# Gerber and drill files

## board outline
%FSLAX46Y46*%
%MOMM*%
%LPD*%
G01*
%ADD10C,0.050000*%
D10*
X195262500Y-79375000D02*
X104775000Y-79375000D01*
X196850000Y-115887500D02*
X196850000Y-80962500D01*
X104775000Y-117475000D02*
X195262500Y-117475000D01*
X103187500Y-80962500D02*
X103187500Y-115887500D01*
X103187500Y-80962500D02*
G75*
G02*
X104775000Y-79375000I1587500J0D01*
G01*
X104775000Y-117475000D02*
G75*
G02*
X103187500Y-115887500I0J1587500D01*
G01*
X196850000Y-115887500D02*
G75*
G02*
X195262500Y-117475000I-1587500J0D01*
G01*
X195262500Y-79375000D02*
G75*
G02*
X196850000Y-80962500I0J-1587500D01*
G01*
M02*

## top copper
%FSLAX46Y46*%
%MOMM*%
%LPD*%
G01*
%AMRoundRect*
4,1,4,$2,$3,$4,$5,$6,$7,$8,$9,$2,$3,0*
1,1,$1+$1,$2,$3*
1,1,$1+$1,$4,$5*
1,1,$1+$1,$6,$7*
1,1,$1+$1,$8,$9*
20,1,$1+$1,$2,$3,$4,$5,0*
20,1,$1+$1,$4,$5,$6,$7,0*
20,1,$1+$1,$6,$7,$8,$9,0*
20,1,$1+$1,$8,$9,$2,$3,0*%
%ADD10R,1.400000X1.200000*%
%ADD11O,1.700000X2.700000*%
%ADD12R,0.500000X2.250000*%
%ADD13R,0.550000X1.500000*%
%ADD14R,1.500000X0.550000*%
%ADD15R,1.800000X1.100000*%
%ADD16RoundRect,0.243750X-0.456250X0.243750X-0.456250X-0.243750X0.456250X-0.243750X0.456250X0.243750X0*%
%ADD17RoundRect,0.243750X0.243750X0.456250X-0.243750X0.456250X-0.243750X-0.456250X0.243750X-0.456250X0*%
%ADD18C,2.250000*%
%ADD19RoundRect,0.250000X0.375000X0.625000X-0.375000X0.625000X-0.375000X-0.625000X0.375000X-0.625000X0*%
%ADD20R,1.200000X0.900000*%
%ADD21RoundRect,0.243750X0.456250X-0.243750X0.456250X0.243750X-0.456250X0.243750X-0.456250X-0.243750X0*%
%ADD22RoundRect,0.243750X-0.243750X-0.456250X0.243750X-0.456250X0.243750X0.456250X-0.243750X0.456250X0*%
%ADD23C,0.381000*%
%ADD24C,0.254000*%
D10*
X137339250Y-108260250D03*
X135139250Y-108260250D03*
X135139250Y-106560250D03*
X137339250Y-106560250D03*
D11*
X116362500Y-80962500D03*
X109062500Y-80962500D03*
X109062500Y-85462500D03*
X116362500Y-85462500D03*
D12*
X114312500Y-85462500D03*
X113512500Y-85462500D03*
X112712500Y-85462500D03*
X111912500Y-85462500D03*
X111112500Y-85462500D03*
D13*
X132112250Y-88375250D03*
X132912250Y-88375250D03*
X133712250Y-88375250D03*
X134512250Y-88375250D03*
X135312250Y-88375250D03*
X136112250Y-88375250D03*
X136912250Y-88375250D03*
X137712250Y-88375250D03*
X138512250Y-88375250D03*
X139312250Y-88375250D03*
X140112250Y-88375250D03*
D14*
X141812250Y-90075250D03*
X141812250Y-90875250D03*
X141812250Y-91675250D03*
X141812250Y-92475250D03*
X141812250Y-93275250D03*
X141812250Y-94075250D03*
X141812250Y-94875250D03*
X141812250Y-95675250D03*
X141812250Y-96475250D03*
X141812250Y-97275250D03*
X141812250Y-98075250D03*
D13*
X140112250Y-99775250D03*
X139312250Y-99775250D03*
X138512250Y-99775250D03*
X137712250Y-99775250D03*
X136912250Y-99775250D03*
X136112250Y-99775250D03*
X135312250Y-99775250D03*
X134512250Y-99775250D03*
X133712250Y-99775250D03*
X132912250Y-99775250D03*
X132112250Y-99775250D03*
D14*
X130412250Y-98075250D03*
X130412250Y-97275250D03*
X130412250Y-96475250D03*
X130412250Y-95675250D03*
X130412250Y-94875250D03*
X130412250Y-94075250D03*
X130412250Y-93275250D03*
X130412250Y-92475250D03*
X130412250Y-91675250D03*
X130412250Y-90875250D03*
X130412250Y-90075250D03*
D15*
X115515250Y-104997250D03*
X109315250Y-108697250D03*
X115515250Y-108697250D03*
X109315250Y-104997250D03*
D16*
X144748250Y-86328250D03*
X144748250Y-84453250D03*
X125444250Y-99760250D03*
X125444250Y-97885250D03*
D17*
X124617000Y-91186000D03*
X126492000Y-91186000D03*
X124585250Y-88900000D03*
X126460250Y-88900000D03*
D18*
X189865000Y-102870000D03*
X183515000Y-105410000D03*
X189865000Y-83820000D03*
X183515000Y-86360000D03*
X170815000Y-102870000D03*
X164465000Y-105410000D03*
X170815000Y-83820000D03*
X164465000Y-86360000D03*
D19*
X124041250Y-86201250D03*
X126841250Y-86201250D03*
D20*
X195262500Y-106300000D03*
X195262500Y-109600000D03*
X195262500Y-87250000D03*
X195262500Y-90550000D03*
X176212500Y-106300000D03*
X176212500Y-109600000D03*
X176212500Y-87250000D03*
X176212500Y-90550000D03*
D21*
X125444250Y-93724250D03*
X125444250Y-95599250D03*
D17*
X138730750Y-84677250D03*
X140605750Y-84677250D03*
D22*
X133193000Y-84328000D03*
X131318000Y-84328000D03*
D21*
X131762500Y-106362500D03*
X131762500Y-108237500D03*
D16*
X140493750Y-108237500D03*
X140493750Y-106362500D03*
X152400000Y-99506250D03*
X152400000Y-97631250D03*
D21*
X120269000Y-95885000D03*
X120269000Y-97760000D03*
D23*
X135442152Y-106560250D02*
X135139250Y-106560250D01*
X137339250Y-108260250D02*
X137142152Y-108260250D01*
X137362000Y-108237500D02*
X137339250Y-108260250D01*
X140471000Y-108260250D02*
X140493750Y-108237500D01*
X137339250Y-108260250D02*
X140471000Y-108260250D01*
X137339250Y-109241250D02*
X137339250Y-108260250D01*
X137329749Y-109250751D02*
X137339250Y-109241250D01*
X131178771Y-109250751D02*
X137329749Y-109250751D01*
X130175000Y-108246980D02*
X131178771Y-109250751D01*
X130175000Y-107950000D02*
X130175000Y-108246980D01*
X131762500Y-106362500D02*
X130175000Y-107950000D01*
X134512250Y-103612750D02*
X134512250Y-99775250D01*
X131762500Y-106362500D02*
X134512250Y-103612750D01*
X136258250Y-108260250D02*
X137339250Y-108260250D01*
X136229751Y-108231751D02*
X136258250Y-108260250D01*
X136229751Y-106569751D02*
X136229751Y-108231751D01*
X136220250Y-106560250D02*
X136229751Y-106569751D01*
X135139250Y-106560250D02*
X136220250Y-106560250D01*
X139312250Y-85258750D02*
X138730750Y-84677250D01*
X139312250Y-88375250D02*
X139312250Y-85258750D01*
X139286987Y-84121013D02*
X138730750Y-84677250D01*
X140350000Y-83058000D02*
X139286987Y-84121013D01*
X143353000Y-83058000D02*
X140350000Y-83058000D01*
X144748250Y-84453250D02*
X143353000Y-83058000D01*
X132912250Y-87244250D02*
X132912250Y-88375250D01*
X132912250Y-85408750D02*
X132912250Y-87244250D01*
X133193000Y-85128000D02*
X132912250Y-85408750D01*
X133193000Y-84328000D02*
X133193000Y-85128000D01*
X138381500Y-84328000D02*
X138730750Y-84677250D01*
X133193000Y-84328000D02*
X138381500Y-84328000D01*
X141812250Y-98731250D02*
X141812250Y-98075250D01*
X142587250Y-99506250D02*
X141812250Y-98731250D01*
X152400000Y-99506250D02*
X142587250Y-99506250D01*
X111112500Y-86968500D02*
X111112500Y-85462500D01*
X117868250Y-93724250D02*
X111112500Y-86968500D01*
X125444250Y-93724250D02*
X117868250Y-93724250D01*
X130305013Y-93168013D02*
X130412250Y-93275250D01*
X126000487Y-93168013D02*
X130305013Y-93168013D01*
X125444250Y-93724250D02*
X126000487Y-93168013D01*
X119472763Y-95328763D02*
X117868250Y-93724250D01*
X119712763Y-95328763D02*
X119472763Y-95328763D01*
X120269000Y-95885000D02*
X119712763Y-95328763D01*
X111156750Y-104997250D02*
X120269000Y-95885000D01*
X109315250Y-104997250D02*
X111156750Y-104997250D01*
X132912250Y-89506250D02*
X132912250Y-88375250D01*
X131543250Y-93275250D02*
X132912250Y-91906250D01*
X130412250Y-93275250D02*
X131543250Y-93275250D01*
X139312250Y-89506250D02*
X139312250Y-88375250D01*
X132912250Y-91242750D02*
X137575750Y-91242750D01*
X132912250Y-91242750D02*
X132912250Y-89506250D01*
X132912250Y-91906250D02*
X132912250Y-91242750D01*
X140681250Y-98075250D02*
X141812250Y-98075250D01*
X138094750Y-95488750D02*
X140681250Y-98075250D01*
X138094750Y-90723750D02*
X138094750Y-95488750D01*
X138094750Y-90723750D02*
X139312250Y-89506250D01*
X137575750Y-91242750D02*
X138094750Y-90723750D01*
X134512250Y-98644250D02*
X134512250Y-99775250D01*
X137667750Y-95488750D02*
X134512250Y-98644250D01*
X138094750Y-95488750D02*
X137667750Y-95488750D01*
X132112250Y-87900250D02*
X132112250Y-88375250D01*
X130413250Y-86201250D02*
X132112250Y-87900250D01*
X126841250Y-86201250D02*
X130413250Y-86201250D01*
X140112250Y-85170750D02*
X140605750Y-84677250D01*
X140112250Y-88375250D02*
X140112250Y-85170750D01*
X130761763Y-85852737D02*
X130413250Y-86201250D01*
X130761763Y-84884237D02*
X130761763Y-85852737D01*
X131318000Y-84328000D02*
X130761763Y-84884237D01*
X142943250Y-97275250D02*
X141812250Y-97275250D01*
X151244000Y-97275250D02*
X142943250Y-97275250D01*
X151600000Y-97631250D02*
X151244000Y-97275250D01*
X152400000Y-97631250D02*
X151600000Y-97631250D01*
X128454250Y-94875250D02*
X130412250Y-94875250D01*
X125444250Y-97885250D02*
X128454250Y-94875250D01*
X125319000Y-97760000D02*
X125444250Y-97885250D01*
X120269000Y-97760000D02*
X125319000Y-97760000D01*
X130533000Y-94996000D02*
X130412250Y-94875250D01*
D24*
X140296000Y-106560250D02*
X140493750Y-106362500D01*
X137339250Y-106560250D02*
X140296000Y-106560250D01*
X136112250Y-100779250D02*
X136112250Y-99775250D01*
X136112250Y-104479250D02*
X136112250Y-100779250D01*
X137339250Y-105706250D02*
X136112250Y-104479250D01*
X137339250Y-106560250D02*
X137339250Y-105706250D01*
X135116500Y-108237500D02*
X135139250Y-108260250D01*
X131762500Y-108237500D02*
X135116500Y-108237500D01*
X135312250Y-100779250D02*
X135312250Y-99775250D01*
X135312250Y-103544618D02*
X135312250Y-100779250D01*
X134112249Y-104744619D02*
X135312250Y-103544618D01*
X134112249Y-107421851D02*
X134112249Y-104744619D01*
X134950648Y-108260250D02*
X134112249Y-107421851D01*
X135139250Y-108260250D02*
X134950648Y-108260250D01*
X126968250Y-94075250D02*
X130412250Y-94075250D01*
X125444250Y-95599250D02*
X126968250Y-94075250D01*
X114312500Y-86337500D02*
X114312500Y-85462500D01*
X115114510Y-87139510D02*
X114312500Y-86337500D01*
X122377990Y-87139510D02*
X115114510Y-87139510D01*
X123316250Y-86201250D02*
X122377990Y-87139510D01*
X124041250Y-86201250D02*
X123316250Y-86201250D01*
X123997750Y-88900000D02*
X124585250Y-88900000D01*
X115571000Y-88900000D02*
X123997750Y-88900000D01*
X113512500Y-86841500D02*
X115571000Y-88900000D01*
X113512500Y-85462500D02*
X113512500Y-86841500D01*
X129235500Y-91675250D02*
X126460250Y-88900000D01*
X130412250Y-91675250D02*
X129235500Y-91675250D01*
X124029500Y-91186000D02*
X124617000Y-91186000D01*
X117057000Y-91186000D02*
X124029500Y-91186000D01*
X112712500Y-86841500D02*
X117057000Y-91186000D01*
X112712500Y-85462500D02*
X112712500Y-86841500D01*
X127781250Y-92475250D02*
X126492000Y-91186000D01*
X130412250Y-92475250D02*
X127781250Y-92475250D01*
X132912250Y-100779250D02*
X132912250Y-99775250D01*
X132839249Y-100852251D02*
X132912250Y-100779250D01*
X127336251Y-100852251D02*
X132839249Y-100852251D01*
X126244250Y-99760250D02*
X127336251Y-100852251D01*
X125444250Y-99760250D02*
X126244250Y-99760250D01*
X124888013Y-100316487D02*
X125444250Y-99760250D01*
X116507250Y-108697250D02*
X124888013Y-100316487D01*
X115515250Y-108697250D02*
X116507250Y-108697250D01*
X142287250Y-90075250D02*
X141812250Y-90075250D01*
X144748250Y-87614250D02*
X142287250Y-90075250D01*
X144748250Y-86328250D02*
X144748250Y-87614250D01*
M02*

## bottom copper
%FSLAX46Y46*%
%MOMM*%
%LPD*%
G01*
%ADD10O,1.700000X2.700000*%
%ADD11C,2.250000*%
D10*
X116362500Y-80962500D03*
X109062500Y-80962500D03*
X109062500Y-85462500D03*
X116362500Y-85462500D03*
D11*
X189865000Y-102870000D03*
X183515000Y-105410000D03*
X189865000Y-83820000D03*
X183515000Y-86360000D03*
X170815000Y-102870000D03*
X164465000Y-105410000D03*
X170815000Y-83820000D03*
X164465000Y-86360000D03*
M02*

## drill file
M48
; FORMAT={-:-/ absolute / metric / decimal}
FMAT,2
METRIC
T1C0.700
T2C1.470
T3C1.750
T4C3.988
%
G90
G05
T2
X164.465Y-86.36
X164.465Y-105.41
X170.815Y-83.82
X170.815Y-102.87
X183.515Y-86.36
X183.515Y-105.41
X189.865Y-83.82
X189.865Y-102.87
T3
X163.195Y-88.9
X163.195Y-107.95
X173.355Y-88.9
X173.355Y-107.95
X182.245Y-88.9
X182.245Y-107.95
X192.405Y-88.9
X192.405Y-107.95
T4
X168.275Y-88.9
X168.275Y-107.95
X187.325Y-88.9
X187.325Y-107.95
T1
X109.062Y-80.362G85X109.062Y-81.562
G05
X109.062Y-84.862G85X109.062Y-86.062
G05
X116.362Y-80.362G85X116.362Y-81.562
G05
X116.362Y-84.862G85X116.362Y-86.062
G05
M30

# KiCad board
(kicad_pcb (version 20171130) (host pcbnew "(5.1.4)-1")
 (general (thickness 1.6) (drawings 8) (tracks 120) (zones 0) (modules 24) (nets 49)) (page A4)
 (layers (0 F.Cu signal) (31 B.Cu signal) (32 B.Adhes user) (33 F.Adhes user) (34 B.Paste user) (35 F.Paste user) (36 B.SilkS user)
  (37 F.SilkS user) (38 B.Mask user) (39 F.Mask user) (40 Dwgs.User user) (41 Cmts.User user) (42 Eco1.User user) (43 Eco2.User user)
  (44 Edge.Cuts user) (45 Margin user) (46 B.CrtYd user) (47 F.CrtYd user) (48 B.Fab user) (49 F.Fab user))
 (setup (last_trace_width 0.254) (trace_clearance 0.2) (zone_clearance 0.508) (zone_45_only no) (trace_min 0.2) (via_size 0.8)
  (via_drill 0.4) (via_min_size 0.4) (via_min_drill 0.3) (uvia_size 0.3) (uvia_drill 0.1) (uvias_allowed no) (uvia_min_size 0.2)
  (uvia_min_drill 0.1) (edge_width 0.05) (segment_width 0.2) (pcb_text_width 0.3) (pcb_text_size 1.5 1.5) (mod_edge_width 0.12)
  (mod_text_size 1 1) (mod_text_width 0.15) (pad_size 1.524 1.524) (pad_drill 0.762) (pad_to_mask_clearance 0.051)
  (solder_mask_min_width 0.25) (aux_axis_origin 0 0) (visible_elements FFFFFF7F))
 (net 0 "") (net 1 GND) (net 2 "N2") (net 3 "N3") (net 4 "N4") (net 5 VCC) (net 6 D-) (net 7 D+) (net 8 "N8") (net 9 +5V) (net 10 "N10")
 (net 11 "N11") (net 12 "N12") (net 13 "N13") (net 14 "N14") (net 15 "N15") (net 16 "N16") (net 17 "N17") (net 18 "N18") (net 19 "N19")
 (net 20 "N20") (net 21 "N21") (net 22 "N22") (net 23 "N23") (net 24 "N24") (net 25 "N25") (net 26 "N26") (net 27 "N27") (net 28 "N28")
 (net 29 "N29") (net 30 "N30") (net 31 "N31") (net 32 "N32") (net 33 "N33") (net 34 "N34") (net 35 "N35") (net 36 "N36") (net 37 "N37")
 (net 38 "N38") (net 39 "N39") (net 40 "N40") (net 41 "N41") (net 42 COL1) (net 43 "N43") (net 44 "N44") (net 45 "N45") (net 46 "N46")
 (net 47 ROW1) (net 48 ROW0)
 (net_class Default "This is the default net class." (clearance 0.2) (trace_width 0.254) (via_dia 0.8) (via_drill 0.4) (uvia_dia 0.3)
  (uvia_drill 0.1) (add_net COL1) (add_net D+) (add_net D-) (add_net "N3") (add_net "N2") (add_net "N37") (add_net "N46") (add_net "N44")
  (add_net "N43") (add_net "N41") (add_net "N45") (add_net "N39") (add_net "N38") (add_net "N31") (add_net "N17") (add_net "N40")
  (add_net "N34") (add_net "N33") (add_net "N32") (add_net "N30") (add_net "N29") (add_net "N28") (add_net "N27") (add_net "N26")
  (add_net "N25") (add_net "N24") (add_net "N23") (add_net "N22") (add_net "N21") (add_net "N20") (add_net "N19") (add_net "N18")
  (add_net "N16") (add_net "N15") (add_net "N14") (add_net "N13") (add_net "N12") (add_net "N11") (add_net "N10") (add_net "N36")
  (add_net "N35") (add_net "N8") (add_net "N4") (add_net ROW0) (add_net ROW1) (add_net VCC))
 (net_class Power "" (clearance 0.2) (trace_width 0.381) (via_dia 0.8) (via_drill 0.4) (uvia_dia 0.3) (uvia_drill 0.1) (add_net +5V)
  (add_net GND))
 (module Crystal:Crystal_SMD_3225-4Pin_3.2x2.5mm (layer F.Cu) (at 136.23925 107.41025 180)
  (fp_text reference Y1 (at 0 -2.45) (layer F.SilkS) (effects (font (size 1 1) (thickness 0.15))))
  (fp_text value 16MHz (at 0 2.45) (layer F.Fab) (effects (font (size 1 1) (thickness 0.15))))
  (pad 4 smd rect (at -1.1 -0.85 180) (size 1.4 1.2) (layers F.Cu F.Paste F.Mask) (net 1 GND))
  (pad 3 smd rect (at 1.1 -0.85 180) (size 1.4 1.2) (layers F.Cu F.Paste F.Mask) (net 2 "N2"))
  (pad 2 smd rect (at 1.1 0.85 180) (size 1.4 1.2) (layers F.Cu F.Paste F.Mask) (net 1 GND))
  (pad 1 smd rect (at -1.1 0.85 180) (size 1.4 1.2) (layers F.Cu F.Paste F.Mask) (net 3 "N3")))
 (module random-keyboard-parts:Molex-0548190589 (layer F.Cu) (at 112.7125 80.9625 270)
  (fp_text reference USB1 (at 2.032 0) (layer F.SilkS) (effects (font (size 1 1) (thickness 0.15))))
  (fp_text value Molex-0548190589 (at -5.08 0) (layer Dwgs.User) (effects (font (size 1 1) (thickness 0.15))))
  (pad 6 thru_hole oval (at 0 -3.65 270) (size 2.7 1.7) (drill oval 1.9 0.7) (layers *.Cu *.Mask) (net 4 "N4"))
  (pad 6 thru_hole oval (at 0 3.65 270) (size 2.7 1.7) (drill oval 1.9 0.7) (layers *.Cu *.Mask) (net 4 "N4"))
  (pad 6 thru_hole oval (at 4.5 3.65 270) (size 2.7 1.7) (drill oval 1.9 0.7) (layers *.Cu *.Mask) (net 4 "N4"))
  (pad 6 thru_hole oval (at 4.5 -3.65 270) (size 2.7 1.7) (drill oval 1.9 0.7) (layers *.Cu *.Mask) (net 4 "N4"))
  (pad 5 smd rect (at 4.5 -1.6 270) (size 2.25 0.5) (layers F.Cu F.Paste F.Mask) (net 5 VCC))
  (pad 4 smd rect (at 4.5 -0.8 270) (size 2.25 0.5) (layers F.Cu F.Paste F.Mask) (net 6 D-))
  (pad 3 smd rect (at 4.5 0 270) (size 2.25 0.5) (layers F.Cu F.Paste F.Mask) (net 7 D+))
  (pad 2 smd rect (at 4.5 0.8 270) (size 2.25 0.5) (layers F.Cu F.Paste F.Mask) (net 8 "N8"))
  (pad 1 smd rect (at 4.5 1.6 270) (size 2.25 0.5) (layers F.Cu F.Paste F.Mask) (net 1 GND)))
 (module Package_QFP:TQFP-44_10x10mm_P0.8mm (layer F.Cu) (at 136.11225 94.07525)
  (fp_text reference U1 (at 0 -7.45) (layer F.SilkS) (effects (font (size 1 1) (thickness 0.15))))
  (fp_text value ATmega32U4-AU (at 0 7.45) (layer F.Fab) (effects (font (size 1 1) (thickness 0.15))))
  (pad 44 smd rect (at -4 -5.7 90) (size 1.5 0.55) (layers F.Cu F.Paste F.Mask) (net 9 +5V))
  (pad 43 smd rect (at -3.2 -5.7 90) (size 1.5 0.55) (layers F.Cu F.Paste F.Mask) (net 1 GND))
  (pad 42 smd rect (at -2.4 -5.7 90) (size 1.5 0.55) (layers F.Cu F.Paste F.Mask) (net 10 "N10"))
  (pad 41 smd rect (at -1.6 -5.7 90) (size 1.5 0.55) (layers F.Cu F.Paste F.Mask) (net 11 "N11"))
  (pad 40 smd rect (at -0.8 -5.7 90) (size 1.5 0.55) (layers F.Cu F.Paste F.Mask) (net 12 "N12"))
  (pad 39 smd rect (at 0 -5.7 90) (size 1.5 0.55) (layers F.Cu F.Paste F.Mask) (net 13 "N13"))
  (pad 38 smd rect (at 0.8 -5.7 90) (size 1.5 0.55) (layers F.Cu F.Paste F.Mask) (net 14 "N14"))
  (pad 37 smd rect (at 1.6 -5.7 90) (size 1.5 0.55) (layers F.Cu F.Paste F.Mask) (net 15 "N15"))
  (pad 36 smd rect (at 2.4 -5.7 90) (size 1.5 0.55) (layers F.Cu F.Paste F.Mask) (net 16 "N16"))
  (pad 35 smd rect (at 3.2 -5.7 90) (size 1.5 0.55) (layers F.Cu F.Paste F.Mask) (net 1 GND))
  (pad 34 smd rect (at 4 -5.7 90) (size 1.5 0.55) (layers F.Cu F.Paste F.Mask) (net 9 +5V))
  (pad 33 smd rect (at 5.7 -4) (size 1.5 0.55) (layers F.Cu F.Paste F.Mask) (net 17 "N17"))
  (pad 32 smd rect (at 5.7 -3.2) (size 1.5 0.55) (layers F.Cu F.Paste F.Mask) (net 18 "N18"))
  (pad 31 smd rect (at 5.7 -2.4) (size 1.5 0.55) (layers F.Cu F.Paste F.Mask) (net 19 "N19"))
  (pad 30 smd rect (at 5.7 -1.6) (size 1.5 0.55) (layers F.Cu F.Paste F.Mask) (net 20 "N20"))
  (pad 29 smd rect (at 5.7 -0.8) (size 1.5 0.55) (layers F.Cu F.Paste F.Mask) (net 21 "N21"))
  (pad 28 smd rect (at 5.7 0) (size 1.5 0.55) (layers F.Cu F.Paste F.Mask) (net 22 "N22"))
  (pad 27 smd rect (at 5.7 0.8) (size 1.5 0.55) (layers F.Cu F.Paste F.Mask) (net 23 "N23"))
  (pad 26 smd rect (at 5.7 1.6) (size 1.5 0.55) (layers F.Cu F.Paste F.Mask) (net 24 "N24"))
  (pad 25 smd rect (at 5.7 2.4) (size 1.5 0.55) (layers F.Cu F.Paste F.Mask) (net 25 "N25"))
  (pad 24 smd rect (at 5.7 3.2) (size 1.5 0.55) (layers F.Cu F.Paste F.Mask) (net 9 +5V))
  (pad 23 smd rect (at 5.7 4) (size 1.5 0.55) (layers F.Cu F.Paste F.Mask) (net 1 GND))
  (pad 22 smd rect (at 4 5.7 90) (size 1.5 0.55) (layers F.Cu F.Paste F.Mask) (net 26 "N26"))
  (pad 21 smd rect (at 3.2 5.7 90) (size 1.5 0.55) (layers F.Cu F.Paste F.Mask) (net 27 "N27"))
  (pad 20 smd rect (at 2.4 5.7 90) (size 1.5 0.55) (layers F.Cu F.Paste F.Mask) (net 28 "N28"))
  (pad 19 smd rect (at 1.6 5.7 90) (size 1.5 0.55) (layers F.Cu F.Paste F.Mask) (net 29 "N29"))
  (pad 18 smd rect (at 0.8 5.7 90) (size 1.5 0.55) (layers F.Cu F.Paste F.Mask) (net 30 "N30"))
  (pad 17 smd rect (at 0 5.7 90) (size 1.5 0.55) (layers F.Cu F.Paste F.Mask) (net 3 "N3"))
  (pad 16 smd rect (at -0.8 5.7 90) (size 1.5 0.55) (layers F.Cu F.Paste F.Mask) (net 2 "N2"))
  (pad 15 smd rect (at -1.6 5.7 90) (size 1.5 0.55) (layers F.Cu F.Paste F.Mask) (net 1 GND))
  (pad 14 smd rect (at -2.4 5.7 90) (size 1.5 0.55) (layers F.Cu F.Paste F.Mask) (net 9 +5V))
  (pad 13 smd rect (at -3.2 5.7 90) (size 1.5 0.55) (layers F.Cu F.Paste F.Mask) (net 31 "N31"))
  (pad 12 smd rect (at -4 5.7 90) (size 1.5 0.55) (layers F.Cu F.Paste F.Mask) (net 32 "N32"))
  (pad 11 smd rect (at -5.7 4) (size 1.5 0.55) (layers F.Cu F.Paste F.Mask) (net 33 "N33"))
  (pad 10 smd rect (at -5.7 3.2) (size 1.5 0.55) (layers F.Cu F.Paste F.Mask) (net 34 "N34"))
  (pad 9 smd rect (at -5.7 2.4) (size 1.5 0.55) (layers F.Cu F.Paste F.Mask) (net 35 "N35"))
  (pad 8 smd rect (at -5.7 1.6) (size 1.5 0.55) (layers F.Cu F.Paste F.Mask) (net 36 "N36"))
  (pad 7 smd rect (at -5.7 0.8) (size 1.5 0.55) (layers F.Cu F.Paste F.Mask) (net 9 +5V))
  (pad 6 smd rect (at -5.7 0) (size 1.5 0.55) (layers F.Cu F.Paste F.Mask) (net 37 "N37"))
  (pad 5 smd rect (at -5.7 -0.8) (size 1.5 0.55) (layers F.Cu F.Paste F.Mask) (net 1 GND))
  (pad 4 smd rect (at -5.7 -1.6) (size 1.5 0.55) (layers F.Cu F.Paste F.Mask) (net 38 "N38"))
  (pad 3 smd rect (at -5.7 -2.4) (size 1.5 0.55) (layers F.Cu F.Paste F.Mask) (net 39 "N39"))
  (pad 2 smd rect (at -5.7 -3.2) (size 1.5 0.55) (layers F.Cu F.Paste F.Mask) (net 9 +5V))
  (pad 1 smd rect (at -5.7 -4) (size 1.5 0.55) (layers F.Cu F.Paste F.Mask) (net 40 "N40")))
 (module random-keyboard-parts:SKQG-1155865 (layer F.Cu) (at 112.41525 106.84725 180)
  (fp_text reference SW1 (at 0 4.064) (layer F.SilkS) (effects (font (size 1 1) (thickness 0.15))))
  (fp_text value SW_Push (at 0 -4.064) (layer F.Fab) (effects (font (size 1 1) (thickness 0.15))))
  (pad 4 smd rect (at -3.1 1.85 180) (size 1.8 1.1) (layers F.Cu F.Paste F.Mask))
  (pad 3 smd rect (at 3.1 -1.85 180) (size 1.8 1.1) (layers F.Cu F.Paste F.Mask))
  (pad 2 smd rect (at -3.1 -1.85 180) (size 1.8 1.1) (layers F.Cu F.Paste F.Mask) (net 31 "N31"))
  (pad 1 smd rect (at 3.1 1.85 180) (size 1.8 1.1) (layers F.Cu F.Paste F.Mask) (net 1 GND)))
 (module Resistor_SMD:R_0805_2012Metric (layer F.Cu) (at 144.74825 85.39075 270)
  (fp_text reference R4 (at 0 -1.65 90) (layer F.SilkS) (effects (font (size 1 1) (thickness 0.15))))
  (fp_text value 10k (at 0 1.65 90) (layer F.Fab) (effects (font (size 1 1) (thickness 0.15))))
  (pad 2 smd roundrect (at 0.9375 0 270) (size 0.975 1.4) (layers F.Cu F.Paste F.Mask) (roundrect_rratio 0.25) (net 17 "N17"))
  (pad 1 smd roundrect (at -0.9375 0 270) (size 0.975 1.4) (layers F.Cu F.Paste F.Mask) (roundrect_rratio 0.25) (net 1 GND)))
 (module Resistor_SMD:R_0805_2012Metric (layer F.Cu) (at 125.44425 98.82275 270)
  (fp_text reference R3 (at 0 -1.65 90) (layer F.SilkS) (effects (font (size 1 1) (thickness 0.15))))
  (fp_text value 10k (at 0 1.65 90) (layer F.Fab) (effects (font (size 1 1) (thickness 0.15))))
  (pad 2 smd roundrect (at 0.9375 0 270) (size 0.975 1.4) (layers F.Cu F.Paste F.Mask) (roundrect_rratio 0.25) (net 31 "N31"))
  (pad 1 smd roundrect (at -0.9375 0 270) (size 0.975 1.4) (layers F.Cu F.Paste F.Mask) (roundrect_rratio 0.25) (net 9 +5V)))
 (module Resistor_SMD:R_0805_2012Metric (layer F.Cu) (at 125.5545 91.186 180)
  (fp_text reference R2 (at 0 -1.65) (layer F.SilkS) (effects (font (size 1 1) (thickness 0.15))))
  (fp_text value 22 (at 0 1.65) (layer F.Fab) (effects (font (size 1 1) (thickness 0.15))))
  (pad 2 smd roundrect (at 0.9375 0 180) (size 0.975 1.4) (layers F.Cu F.Paste F.Mask) (roundrect_rratio 0.25) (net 7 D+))
  (pad 1 smd roundrect (at -0.9375 0 180) (size 0.975 1.4) (layers F.Cu F.Paste F.Mask) (roundrect_rratio 0.25) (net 38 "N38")))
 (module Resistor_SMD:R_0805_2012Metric (layer F.Cu) (at 125.52275 88.9 180)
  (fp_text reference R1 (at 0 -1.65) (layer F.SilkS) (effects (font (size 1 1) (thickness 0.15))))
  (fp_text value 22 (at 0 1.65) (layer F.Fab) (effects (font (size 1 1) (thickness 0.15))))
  (pad 2 smd roundrect (at 0.9375 0 180) (size 0.975 1.4) (layers F.Cu F.Paste F.Mask) (roundrect_rratio 0.25) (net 6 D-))
  (pad 1 smd roundrect (at -0.9375 0 180) (size 0.975 1.4) (layers F.Cu F.Paste F.Mask) (roundrect_rratio 0.25) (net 39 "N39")))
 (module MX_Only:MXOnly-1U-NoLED (layer F.Cu) (at 187.325 107.95)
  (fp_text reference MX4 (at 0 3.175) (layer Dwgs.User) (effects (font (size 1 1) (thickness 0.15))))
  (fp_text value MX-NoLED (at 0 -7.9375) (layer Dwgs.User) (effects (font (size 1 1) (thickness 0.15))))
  (pad 2 thru_hole circle (at 2.54 -5.08) (size 2.25 2.25) (drill 1.47) (layers *.Cu B.Mask) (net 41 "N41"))
  (pad "" np_thru_hole circle (at 0 0) (size 3.9878 3.9878) (drill 3.9878) (layers *.Cu *.Mask))
  (pad 1 thru_hole circle (at -3.81 -2.54) (size 2.25 2.25) (drill 1.47) (layers *.Cu B.Mask) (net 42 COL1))
  (pad "" np_thru_hole circle (at -5.08 0 48.0996) (size 1.75 1.75) (drill 1.75) (layers *.Cu *.Mask))
  (pad "" np_thru_hole circle (at 5.08 0 48.0996) (size 1.75 1.75) (drill 1.75) (layers *.Cu *.Mask)))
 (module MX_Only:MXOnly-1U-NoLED (layer F.Cu) (at 187.325 88.9)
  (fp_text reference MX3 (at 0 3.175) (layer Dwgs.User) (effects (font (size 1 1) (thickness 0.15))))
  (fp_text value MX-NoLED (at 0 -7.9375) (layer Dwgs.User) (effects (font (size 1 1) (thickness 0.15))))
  (pad 2 thru_hole circle (at 2.54 -5.08) (size 2.25 2.25) (drill 1.47) (layers *.Cu B.Mask) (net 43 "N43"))
  (pad "" np_thru_hole circle (at 0 0) (size 3.9878 3.9878) (drill 3.9878) (layers *.Cu *.Mask))
  (pad 1 thru_hole circle (at -3.81 -2.54) (size 2.25 2.25) (drill 1.47) (layers *.Cu B.Mask) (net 42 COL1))
  (pad "" np_thru_hole circle (at -5.08 0 48.0996) (size 1.75 1.75) (drill 1.75) (layers *.Cu *.Mask))
  (pad "" np_thru_hole circle (at 5.08 0 48.0996) (size 1.75 1.75) (drill 1.75) (layers *.Cu *.Mask)))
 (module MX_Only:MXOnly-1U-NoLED (layer F.Cu) (at 168.275 107.95)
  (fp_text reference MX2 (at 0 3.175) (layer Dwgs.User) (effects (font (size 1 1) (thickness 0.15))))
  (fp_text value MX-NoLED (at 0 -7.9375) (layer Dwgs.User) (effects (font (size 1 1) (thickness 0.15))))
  (pad 2 thru_hole circle (at 2.54 -5.08) (size 2.25 2.25) (drill 1.47) (layers *.Cu B.Mask) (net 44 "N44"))
  (pad "" np_thru_hole circle (at 0 0) (size 3.9878 3.9878) (drill 3.9878) (layers *.Cu *.Mask))
  (pad 1 thru_hole circle (at -3.81 -2.54) (size 2.25 2.25) (drill 1.47) (layers *.Cu B.Mask) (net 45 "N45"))
  (pad "" np_thru_hole circle (at -5.08 0 48.0996) (size 1.75 1.75) (drill 1.75) (layers *.Cu *.Mask))
  (pad "" np_thru_hole circle (at 5.08 0 48.0996) (size 1.75 1.75) (drill 1.75) (layers *.Cu *.Mask)))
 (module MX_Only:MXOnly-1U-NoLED (layer F.Cu) (at 168.275 88.9)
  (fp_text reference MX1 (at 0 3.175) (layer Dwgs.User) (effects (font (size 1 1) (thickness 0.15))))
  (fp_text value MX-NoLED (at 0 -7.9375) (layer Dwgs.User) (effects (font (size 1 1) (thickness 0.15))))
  (pad 2 thru_hole circle (at 2.54 -5.08) (size 2.25 2.25) (drill 1.47) (layers *.Cu B.Mask) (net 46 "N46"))
  (pad "" np_thru_hole circle (at 0 0) (size 3.9878 3.9878) (drill 3.9878) (layers *.Cu *.Mask))
  (pad 1 thru_hole circle (at -3.81 -2.54) (size 2.25 2.25) (drill 1.47) (layers *.Cu B.Mask) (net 45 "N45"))
  (pad "" np_thru_hole circle (at -5.08 0 48.0996) (size 1.75 1.75) (drill 1.75) (layers *.Cu *.Mask))
  (pad "" np_thru_hole circle (at 5.08 0 48.0996) (size 1.75 1.75) (drill 1.75) (layers *.Cu *.Mask)))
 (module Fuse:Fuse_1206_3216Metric (layer F.Cu) (at 125.44125 86.20125 180)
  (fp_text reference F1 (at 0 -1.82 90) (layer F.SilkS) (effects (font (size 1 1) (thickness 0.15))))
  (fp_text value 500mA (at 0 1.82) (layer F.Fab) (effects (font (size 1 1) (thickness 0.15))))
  (pad 2 smd roundrect (at 1.4 0 180) (size 1.25 1.75) (layers F.Cu F.Paste F.Mask) (roundrect_rratio 0.2) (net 5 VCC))
  (pad 1 smd roundrect (at -1.4 0 180) (size 1.25 1.75) (layers F.Cu F.Paste F.Mask) (roundrect_rratio 0.2) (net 9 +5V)))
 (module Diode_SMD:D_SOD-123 (layer F.Cu) (at 195.2625 107.95 90)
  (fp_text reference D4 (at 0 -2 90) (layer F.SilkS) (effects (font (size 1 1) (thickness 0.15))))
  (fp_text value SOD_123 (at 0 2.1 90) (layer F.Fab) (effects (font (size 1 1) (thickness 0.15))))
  (pad 2 smd rect (at 1.65 0 90) (size 0.9 1.2) (layers F.Cu F.Paste F.Mask) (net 41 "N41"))
  (pad 1 smd rect (at -1.65 0 90) (size 0.9 1.2) (layers F.Cu F.Paste F.Mask) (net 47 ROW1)))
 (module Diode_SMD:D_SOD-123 (layer F.Cu) (at 195.2625 88.9 90)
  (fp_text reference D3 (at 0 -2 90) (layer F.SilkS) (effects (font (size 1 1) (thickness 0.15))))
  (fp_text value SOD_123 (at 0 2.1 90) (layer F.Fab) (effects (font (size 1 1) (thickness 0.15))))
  (pad 2 smd rect (at 1.65 0 90) (size 0.9 1.2) (layers F.Cu F.Paste F.Mask) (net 43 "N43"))
  (pad 1 smd rect (at -1.65 0 90) (size 0.9 1.2) (layers F.Cu F.Paste F.Mask) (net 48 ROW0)))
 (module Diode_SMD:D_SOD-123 (layer F.Cu) (at 176.2125 107.95 90)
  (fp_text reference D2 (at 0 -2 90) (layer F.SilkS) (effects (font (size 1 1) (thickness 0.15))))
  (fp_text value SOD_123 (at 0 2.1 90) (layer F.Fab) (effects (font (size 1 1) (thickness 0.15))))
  (pad 2 smd rect (at 1.65 0 90) (size 0.9 1.2) (layers F.Cu F.Paste F.Mask) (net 44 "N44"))
  (pad 1 smd rect (at -1.65 0 90) (size 0.9 1.2) (layers F.Cu F.Paste F.Mask) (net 47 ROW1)))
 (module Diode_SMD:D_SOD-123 (layer F.Cu) (at 176.2125 88.9 90)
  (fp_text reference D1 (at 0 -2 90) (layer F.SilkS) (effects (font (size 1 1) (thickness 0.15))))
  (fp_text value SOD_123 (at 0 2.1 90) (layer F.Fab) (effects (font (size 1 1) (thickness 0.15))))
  (pad 2 smd rect (at 1.65 0 90) (size 0.9 1.2) (layers F.Cu F.Paste F.Mask) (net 46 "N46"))
  (pad 1 smd rect (at -1.65 0 90) (size 0.9 1.2) (layers F.Cu F.Paste F.Mask) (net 48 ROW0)))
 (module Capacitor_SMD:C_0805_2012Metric (layer F.Cu) (at 125.44425 94.66175 90)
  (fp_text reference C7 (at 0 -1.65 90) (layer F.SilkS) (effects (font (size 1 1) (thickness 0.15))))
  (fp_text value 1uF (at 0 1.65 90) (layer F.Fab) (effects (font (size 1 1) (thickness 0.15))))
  (pad 2 smd roundrect (at 0.9375 0 90) (size 0.975 1.4) (layers F.Cu F.Paste F.Mask) (roundrect_rratio 0.25) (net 1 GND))
  (pad 1 smd roundrect (at -0.9375 0 90) (size 0.975 1.4) (layers F.Cu F.Paste F.Mask) (roundrect_rratio 0.25) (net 37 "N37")))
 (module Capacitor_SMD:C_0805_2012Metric (layer F.Cu) (at 139.66825 84.67725 180)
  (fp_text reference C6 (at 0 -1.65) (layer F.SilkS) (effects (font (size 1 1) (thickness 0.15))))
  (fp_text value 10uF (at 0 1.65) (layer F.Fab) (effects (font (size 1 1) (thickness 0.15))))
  (pad 2 smd roundrect (at 0.9375 0 180) (size 0.975 1.4) (layers F.Cu F.Paste F.Mask) (roundrect_rratio 0.25) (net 1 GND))
  (pad 1 smd roundrect (at -0.9375 0 180) (size 0.975 1.4) (layers F.Cu F.Paste F.Mask) (roundrect_rratio 0.25) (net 9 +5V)))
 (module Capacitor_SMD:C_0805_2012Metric (layer F.Cu) (at 132.2555 84.328)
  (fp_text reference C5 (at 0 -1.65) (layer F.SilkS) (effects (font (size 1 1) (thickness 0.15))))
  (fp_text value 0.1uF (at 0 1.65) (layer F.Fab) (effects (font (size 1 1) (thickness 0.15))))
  (pad 2 smd roundrect (at 0.9375 0) (size 0.975 1.4) (layers F.Cu F.Paste F.Mask) (roundrect_rratio 0.25) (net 1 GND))
  (pad 1 smd roundrect (at -0.9375 0) (size 0.975 1.4) (layers F.Cu F.Paste F.Mask) (roundrect_rratio 0.25) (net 9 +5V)))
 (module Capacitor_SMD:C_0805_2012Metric (layer F.Cu) (at 131.7625 107.3 90)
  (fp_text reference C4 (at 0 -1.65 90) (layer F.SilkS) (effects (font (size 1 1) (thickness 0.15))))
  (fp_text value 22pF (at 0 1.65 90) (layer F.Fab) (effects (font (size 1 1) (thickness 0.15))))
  (pad 2 smd roundrect (at 0.9375 0 90) (size 0.975 1.4) (layers F.Cu F.Paste F.Mask) (roundrect_rratio 0.25) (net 1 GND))
  (pad 1 smd roundrect (at -0.9375 0 90) (size 0.975 1.4) (layers F.Cu F.Paste F.Mask) (roundrect_rratio 0.25) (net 2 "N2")))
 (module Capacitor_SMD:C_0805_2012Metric (layer F.Cu) (at 140.49375 107.3 270)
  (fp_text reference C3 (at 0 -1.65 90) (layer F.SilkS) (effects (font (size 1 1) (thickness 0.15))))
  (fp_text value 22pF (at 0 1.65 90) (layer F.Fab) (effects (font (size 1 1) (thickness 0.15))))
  (pad 2 smd roundrect (at 0.9375 0 270) (size 0.975 1.4) (layers F.Cu F.Paste F.Mask) (roundrect_rratio 0.25) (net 1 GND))
  (pad 1 smd roundrect (at -0.9375 0 270) (size 0.975 1.4) (layers F.Cu F.Paste F.Mask) (roundrect_rratio 0.25) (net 3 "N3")))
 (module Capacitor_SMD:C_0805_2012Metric (layer F.Cu) (at 152.4 98.56875 270)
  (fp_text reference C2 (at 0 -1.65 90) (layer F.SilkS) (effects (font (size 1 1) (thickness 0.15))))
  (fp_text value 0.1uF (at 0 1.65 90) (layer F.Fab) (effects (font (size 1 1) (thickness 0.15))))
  (pad 2 smd roundrect (at 0.9375 0 270) (size 0.975 1.4) (layers F.Cu F.Paste F.Mask) (roundrect_rratio 0.25) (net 1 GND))
  (pad 1 smd roundrect (at -0.9375 0 270) (size 0.975 1.4) (layers F.Cu F.Paste F.Mask) (roundrect_rratio 0.25) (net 9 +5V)))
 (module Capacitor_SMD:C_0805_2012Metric (layer F.Cu) (at 120.269 96.8225 90)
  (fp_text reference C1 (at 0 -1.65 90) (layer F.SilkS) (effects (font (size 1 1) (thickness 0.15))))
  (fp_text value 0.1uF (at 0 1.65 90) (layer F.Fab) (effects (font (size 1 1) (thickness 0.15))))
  (pad 2 smd roundrect (at 0.9375 0 90) (size 0.975 1.4) (layers F.Cu F.Paste F.Mask) (roundrect_rratio 0.25) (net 1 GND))
  (pad 1 smd roundrect (at -0.9375 0 90) (size 0.975 1.4) (layers F.Cu F.Paste F.Mask) (roundrect_rratio 0.25) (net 9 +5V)))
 (gr_line (start 195.2625 79.375) (end 104.775 79.375) (layer Edge.Cuts) (width 0.05))
 (gr_line (start 196.85 115.8875) (end 196.85 80.9625) (layer Edge.Cuts) (width 0.05))
 (gr_line (start 104.775 117.475) (end 195.2625 117.475) (layer Edge.Cuts) (width 0.05))
 (gr_line (start 103.1875 80.9625) (end 103.1875 115.8875) (layer Edge.Cuts) (width 0.05))
 (gr_arc (start 104.775 80.9625) (end 104.775 79.375) (angle -90) (layer Edge.Cuts) (width 0.05))
 (gr_arc (start 104.775 115.8875) (end 103.1875 115.8875) (angle -90) (layer Edge.Cuts) (width 0.05))
 (gr_arc (start 195.2625 115.8875) (end 195.2625 117.475) (angle -90) (layer Edge.Cuts) (width 0.05))
 (gr_arc (start 195.2625 80.9625) (end 196.85 80.9625) (angle -90) (layer Edge.Cuts) (width 0.05))
 (segment (start 135.442152 106.56025) (end 135.13925 106.56025) (width 0.381) (layer F.Cu) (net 1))
 (segment (start 137.33925 108.26025) (end 137.142152 108.26025) (width 0.381) (layer F.Cu) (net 1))
 (segment (start 137.362 108.2375) (end 137.33925 108.26025) (width 0.381) (layer F.Cu) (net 1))
 (segment (start 140.471 108.26025) (end 140.49375 108.2375) (width 0.381) (layer F.Cu) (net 1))
 (segment (start 137.33925 108.26025) (end 140.471 108.26025) (width 0.381) (layer F.Cu) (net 1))
 (segment (start 137.33925 109.24125) (end 137.33925 108.26025) (width 0.381) (layer F.Cu) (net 1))
 (segment (start 137.329749 109.250751) (end 137.33925 109.24125) (width 0.381) (layer F.Cu) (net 1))
 (segment (start 131.178771 109.250751) (end 137.329749 109.250751) (width 0.381) (layer F.Cu) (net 1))
 (segment (start 130.175 108.24698) (end 131.178771 109.250751) (width 0.381) (layer F.Cu) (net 1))
 (segment (start 130.175 107.95) (end 130.175 108.24698) (width 0.381) (layer F.Cu) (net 1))
 (segment (start 131.7625 106.3625) (end 130.175 107.95) (width 0.381) (layer F.Cu) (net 1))
 (segment (start 134.51225 103.61275) (end 134.51225 99.77525) (width 0.381) (layer F.Cu) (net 1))
 (segment (start 131.7625 106.3625) (end 134.51225 103.61275) (width 0.381) (layer F.Cu) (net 1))
 (segment (start 136.25825 108.26025) (end 137.33925 108.26025) (width 0.381) (layer F.Cu) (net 1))
 (segment (start 136.229751 108.231751) (end 136.25825 108.26025) (width 0.381) (layer F.Cu) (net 1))
 (segment (start 136.229751 106.569751) (end 136.229751 108.231751) (width 0.381) (layer F.Cu) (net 1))
 (segment (start 136.22025 106.56025) (end 136.229751 106.569751) (width 0.381) (layer F.Cu) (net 1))
 (segment (start 135.13925 106.56025) (end 136.22025 106.56025) (width 0.381) (layer F.Cu) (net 1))
 (segment (start 139.31225 85.25875) (end 138.73075 84.67725) (width 0.381) (layer F.Cu) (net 1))
 (segment (start 139.31225 88.37525) (end 139.31225 85.25875) (width 0.381) (layer F.Cu) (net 1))
 (segment (start 139.286987 84.121013) (end 138.73075 84.67725) (width 0.381) (layer F.Cu) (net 1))
 (segment (start 140.35 83.058) (end 139.286987 84.121013) (width 0.381) (layer F.Cu) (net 1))
 (segment (start 143.353 83.058) (end 140.35 83.058) (width 0.381) (layer F.Cu) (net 1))
 (segment (start 144.74825 84.45325) (end 143.353 83.058) (width 0.381) (layer F.Cu) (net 1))
 (segment (start 132.91225 87.24425) (end 132.91225 88.37525) (width 0.381) (layer F.Cu) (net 1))
 (segment (start 132.91225 85.40875) (end 132.91225 87.24425) (width 0.381) (layer F.Cu) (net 1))
 (segment (start 133.193 85.128) (end 132.91225 85.40875) (width 0.381) (layer F.Cu) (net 1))
 (segment (start 133.193 84.328) (end 133.193 85.128) (width 0.381) (layer F.Cu) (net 1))
 (segment (start 138.3815 84.328) (end 138.73075 84.67725) (width 0.381) (layer F.Cu) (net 1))
 (segment (start 133.193 84.328) (end 138.3815 84.328) (width 0.381) (layer F.Cu) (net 1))
 (segment (start 141.81225 98.73125) (end 141.81225 98.07525) (width 0.381) (layer F.Cu) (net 1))
 (segment (start 142.58725 99.50625) (end 141.81225 98.73125) (width 0.381) (layer F.Cu) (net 1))
 (segment (start 152.4 99.50625) (end 142.58725 99.50625) (width 0.381) (layer F.Cu) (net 1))
 (segment (start 111.1125 86.9685) (end 111.1125 85.4625) (width 0.381) (layer F.Cu) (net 1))
 (segment (start 117.86825 93.72425) (end 111.1125 86.9685) (width 0.381) (layer F.Cu) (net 1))
 (segment (start 125.44425 93.72425) (end 117.86825 93.72425) (width 0.381) (layer F.Cu) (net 1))
 (segment (start 130.305013 93.168013) (end 130.41225 93.27525) (width 0.381) (layer F.Cu) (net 1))
 (segment (start 126.000487 93.168013) (end 130.305013 93.168013) (width 0.381) (layer F.Cu) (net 1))
 (segment (start 125.44425 93.72425) (end 126.000487 93.168013) (width 0.381) (layer F.Cu) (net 1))
 (segment (start 119.472763 95.328763) (end 117.86825 93.72425) (width 0.381) (layer F.Cu) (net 1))
 (segment (start 119.712763 95.328763) (end 119.472763 95.328763) (width 0.381) (layer F.Cu) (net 1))
 (segment (start 120.269 95.885) (end 119.712763 95.328763) (width 0.381) (layer F.Cu) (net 1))
 (segment (start 111.15675 104.99725) (end 120.269 95.885) (width 0.381) (layer F.Cu) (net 1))
 (segment (start 109.31525 104.99725) (end 111.15675 104.99725) (width 0.381) (layer F.Cu) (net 1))
 (segment (start 132.91225 89.50625) (end 132.91225 88.37525) (width 0.381) (layer F.Cu) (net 1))
 (segment (start 131.54325 93.27525) (end 132.91225 91.90625) (width 0.381) (layer F.Cu) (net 1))
 (segment (start 130.41225 93.27525) (end 131.54325 93.27525) (width 0.381) (layer F.Cu) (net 1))
 (segment (start 139.31225 89.50625) (end 139.31225 88.37525) (width 0.381) (layer F.Cu) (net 1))
 (segment (start 132.91225 91.24275) (end 137.57575 91.24275) (width 0.381) (layer F.Cu) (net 1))
 (segment (start 132.91225 91.24275) (end 132.91225 89.50625) (width 0.381) (layer F.Cu) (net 1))
 (segment (start 132.91225 91.90625) (end 132.91225 91.24275) (width 0.381) (layer F.Cu) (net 1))
 (segment (start 140.68125 98.07525) (end 141.81225 98.07525) (width 0.381) (layer F.Cu) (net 1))
 (segment (start 138.09475 95.48875) (end 140.68125 98.07525) (width 0.381) (layer F.Cu) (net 1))
 (segment (start 138.09475 90.72375) (end 138.09475 95.48875) (width 0.381) (layer F.Cu) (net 1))
 (segment (start 138.09475 90.72375) (end 139.31225 89.50625) (width 0.381) (layer F.Cu) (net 1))
 (segment (start 137.57575 91.24275) (end 138.09475 90.72375) (width 0.381) (layer F.Cu) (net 1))
 (segment (start 134.51225 98.64425) (end 134.51225 99.77525) (width 0.381) (layer F.Cu) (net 1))
 (segment (start 137.66775 95.48875) (end 134.51225 98.64425) (width 0.381) (layer F.Cu) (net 1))
 (segment (start 138.09475 95.48875) (end 137.66775 95.48875) (width 0.381) (layer F.Cu) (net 1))
 (segment (start 132.11225 87.90025) (end 132.11225 88.37525) (width 0.381) (layer F.Cu) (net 9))
 (segment (start 130.41325 86.20125) (end 132.11225 87.90025) (width 0.381) (layer F.Cu) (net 9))
 (segment (start 126.84125 86.20125) (end 130.41325 86.20125) (width 0.381) (layer F.Cu) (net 9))
 (segment (start 140.11225 85.17075) (end 140.60575 84.67725) (width 0.381) (layer F.Cu) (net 9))
 (segment (start 140.11225 88.37525) (end 140.11225 85.17075) (width 0.381) (layer F.Cu) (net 9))
 (segment (start 130.761763 85.852737) (end 130.41325 86.20125) (width 0.381) (layer F.Cu) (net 9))
 (segment (start 130.761763 84.884237) (end 130.761763 85.852737) (width 0.381) (layer F.Cu) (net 9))
 (segment (start 131.318 84.328) (end 130.761763 84.884237) (width 0.381) (layer F.Cu) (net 9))
 (segment (start 142.94325 97.27525) (end 141.81225 97.27525) (width 0.381) (layer F.Cu) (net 9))
 (segment (start 151.244 97.27525) (end 142.94325 97.27525) (width 0.381) (layer F.Cu) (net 9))
 (segment (start 151.6 97.63125) (end 151.244 97.27525) (width 0.381) (layer F.Cu) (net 9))
 (segment (start 152.4 97.63125) (end 151.6 97.63125) (width 0.381) (layer F.Cu) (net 9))
 (segment (start 128.45425 94.87525) (end 130.41225 94.87525) (width 0.381) (layer F.Cu) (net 9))
 (segment (start 125.44425 97.88525) (end 128.45425 94.87525) (width 0.381) (layer F.Cu) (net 9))
 (segment (start 125.319 97.76) (end 125.44425 97.88525) (width 0.381) (layer F.Cu) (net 9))
 (segment (start 120.269 97.76) (end 125.319 97.76) (width 0.381) (layer F.Cu) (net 9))
 (segment (start 130.533 94.996) (end 130.41225 94.87525) (width 0.381) (layer F.Cu) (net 9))
 (segment (start 140.296 106.56025) (end 140.49375 106.3625) (width 0.254) (layer F.Cu) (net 3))
 (segment (start 137.33925 106.56025) (end 140.296 106.56025) (width 0.254) (layer F.Cu) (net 3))
 (segment (start 136.11225 100.77925) (end 136.11225 99.77525) (width 0.254) (layer F.Cu) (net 3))
 (segment (start 136.11225 104.47925) (end 136.11225 100.77925) (width 0.254) (layer F.Cu) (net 3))
 (segment (start 137.33925 105.70625) (end 136.11225 104.47925) (width 0.254) (layer F.Cu) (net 3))
 (segment (start 137.33925 106.56025) (end 137.33925 105.70625) (width 0.254) (layer F.Cu) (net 3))
 (segment (start 135.1165 108.2375) (end 135.13925 108.26025) (width 0.254) (layer F.Cu) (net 2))
 (segment (start 131.7625 108.2375) (end 135.1165 108.2375) (width 0.254) (layer F.Cu) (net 2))
 (segment (start 135.31225 100.77925) (end 135.31225 99.77525) (width 0.254) (layer F.Cu) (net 2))
 (segment (start 135.31225 103.544618) (end 135.31225 100.77925) (width 0.254) (layer F.Cu) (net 2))
 (segment (start 134.112249 104.744619) (end 135.31225 103.544618) (width 0.254) (layer F.Cu) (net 2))
 (segment (start 134.112249 107.421851) (end 134.112249 104.744619) (width 0.254) (layer F.Cu) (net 2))
 (segment (start 134.950648 108.26025) (end 134.112249 107.421851) (width 0.254) (layer F.Cu) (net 2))
 (segment (start 135.13925 108.26025) (end 134.950648 108.26025) (width 0.254) (layer F.Cu) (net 2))
 (segment (start 126.96825 94.07525) (end 130.41225 94.07525) (width 0.254) (layer F.Cu) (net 37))
 (segment (start 125.44425 95.59925) (end 126.96825 94.07525) (width 0.254) (layer F.Cu) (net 37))
 (segment (start 114.3125 86.3375) (end 114.3125 85.4625) (width 0.254) (layer F.Cu) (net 5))
 (segment (start 115.11451 87.13951) (end 114.3125 86.3375) (width 0.254) (layer F.Cu) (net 5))
 (segment (start 122.37799 87.13951) (end 115.11451 87.13951) (width 0.254) (layer F.Cu) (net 5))
 (segment (start 123.31625 86.20125) (end 122.37799 87.13951) (width 0.254) (layer F.Cu) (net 5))
 (segment (start 124.04125 86.20125) (end 123.31625 86.20125) (width 0.254) (layer F.Cu) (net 5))
 (segment (start 123.99775 88.9) (end 124.58525 88.9) (width 0.254) (layer F.Cu) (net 6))
 (segment (start 115.571 88.9) (end 123.99775 88.9) (width 0.254) (layer F.Cu) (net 6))
 (segment (start 113.5125 86.8415) (end 115.571 88.9) (width 0.254) (layer F.Cu) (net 6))
 (segment (start 113.5125 85.4625) (end 113.5125 86.8415) (width 0.254) (layer F.Cu) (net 6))
 (segment (start 129.2355 91.67525) (end 126.46025 88.9) (width 0.254) (layer F.Cu) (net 39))
 (segment (start 130.41225 91.67525) (end 129.2355 91.67525) (width 0.254) (layer F.Cu) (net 39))
 (segment (start 124.0295 91.186) (end 124.617 91.186) (width 0.254) (layer F.Cu) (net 7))
 (segment (start 117.057 91.186) (end 124.0295 91.186) (width 0.254) (layer F.Cu) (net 7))
 (segment (start 112.7125 86.8415) (end 117.057 91.186) (width 0.254) (layer F.Cu) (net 7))
 (segment (start 112.7125 85.4625) (end 112.7125 86.8415) (width 0.254) (layer F.Cu) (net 7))
 (segment (start 127.78125 92.47525) (end 126.492 91.186) (width 0.254) (layer F.Cu) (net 38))
 (segment (start 130.41225 92.47525) (end 127.78125 92.47525) (width 0.254) (layer F.Cu) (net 38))
 (segment (start 132.91225 100.77925) (end 132.91225 99.77525) (width 0.254) (layer F.Cu) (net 31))
 (segment (start 132.839249 100.852251) (end 132.91225 100.77925) (width 0.254) (layer F.Cu) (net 31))
 (segment (start 127.336251 100.852251) (end 132.839249 100.852251) (width 0.254) (layer F.Cu) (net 31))
 (segment (start 126.24425 99.76025) (end 127.336251 100.852251) (width 0.254) (layer F.Cu) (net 31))
 (segment (start 125.44425 99.76025) (end 126.24425 99.76025) (width 0.254) (layer F.Cu) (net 31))
 (segment (start 124.888013 100.316487) (end 125.44425 99.76025) (width 0.254) (layer F.Cu) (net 31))
 (segment (start 116.50725 108.69725) (end 124.888013 100.316487) (width 0.254) (layer F.Cu) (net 31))
 (segment (start 115.51525 108.69725) (end 116.50725 108.69725) (width 0.254) (layer F.Cu) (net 31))
 (segment (start 142.28725 90.07525) (end 141.81225 90.07525) (width 0.254) (layer F.Cu) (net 17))
 (segment (start 144.74825 87.61425) (end 142.28725 90.07525) (width 0.254) (layer F.Cu) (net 17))
 (segment (start 144.74825 86.32825) (end 144.74825 87.61425) (width 0.254) (layer F.Cu) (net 17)))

